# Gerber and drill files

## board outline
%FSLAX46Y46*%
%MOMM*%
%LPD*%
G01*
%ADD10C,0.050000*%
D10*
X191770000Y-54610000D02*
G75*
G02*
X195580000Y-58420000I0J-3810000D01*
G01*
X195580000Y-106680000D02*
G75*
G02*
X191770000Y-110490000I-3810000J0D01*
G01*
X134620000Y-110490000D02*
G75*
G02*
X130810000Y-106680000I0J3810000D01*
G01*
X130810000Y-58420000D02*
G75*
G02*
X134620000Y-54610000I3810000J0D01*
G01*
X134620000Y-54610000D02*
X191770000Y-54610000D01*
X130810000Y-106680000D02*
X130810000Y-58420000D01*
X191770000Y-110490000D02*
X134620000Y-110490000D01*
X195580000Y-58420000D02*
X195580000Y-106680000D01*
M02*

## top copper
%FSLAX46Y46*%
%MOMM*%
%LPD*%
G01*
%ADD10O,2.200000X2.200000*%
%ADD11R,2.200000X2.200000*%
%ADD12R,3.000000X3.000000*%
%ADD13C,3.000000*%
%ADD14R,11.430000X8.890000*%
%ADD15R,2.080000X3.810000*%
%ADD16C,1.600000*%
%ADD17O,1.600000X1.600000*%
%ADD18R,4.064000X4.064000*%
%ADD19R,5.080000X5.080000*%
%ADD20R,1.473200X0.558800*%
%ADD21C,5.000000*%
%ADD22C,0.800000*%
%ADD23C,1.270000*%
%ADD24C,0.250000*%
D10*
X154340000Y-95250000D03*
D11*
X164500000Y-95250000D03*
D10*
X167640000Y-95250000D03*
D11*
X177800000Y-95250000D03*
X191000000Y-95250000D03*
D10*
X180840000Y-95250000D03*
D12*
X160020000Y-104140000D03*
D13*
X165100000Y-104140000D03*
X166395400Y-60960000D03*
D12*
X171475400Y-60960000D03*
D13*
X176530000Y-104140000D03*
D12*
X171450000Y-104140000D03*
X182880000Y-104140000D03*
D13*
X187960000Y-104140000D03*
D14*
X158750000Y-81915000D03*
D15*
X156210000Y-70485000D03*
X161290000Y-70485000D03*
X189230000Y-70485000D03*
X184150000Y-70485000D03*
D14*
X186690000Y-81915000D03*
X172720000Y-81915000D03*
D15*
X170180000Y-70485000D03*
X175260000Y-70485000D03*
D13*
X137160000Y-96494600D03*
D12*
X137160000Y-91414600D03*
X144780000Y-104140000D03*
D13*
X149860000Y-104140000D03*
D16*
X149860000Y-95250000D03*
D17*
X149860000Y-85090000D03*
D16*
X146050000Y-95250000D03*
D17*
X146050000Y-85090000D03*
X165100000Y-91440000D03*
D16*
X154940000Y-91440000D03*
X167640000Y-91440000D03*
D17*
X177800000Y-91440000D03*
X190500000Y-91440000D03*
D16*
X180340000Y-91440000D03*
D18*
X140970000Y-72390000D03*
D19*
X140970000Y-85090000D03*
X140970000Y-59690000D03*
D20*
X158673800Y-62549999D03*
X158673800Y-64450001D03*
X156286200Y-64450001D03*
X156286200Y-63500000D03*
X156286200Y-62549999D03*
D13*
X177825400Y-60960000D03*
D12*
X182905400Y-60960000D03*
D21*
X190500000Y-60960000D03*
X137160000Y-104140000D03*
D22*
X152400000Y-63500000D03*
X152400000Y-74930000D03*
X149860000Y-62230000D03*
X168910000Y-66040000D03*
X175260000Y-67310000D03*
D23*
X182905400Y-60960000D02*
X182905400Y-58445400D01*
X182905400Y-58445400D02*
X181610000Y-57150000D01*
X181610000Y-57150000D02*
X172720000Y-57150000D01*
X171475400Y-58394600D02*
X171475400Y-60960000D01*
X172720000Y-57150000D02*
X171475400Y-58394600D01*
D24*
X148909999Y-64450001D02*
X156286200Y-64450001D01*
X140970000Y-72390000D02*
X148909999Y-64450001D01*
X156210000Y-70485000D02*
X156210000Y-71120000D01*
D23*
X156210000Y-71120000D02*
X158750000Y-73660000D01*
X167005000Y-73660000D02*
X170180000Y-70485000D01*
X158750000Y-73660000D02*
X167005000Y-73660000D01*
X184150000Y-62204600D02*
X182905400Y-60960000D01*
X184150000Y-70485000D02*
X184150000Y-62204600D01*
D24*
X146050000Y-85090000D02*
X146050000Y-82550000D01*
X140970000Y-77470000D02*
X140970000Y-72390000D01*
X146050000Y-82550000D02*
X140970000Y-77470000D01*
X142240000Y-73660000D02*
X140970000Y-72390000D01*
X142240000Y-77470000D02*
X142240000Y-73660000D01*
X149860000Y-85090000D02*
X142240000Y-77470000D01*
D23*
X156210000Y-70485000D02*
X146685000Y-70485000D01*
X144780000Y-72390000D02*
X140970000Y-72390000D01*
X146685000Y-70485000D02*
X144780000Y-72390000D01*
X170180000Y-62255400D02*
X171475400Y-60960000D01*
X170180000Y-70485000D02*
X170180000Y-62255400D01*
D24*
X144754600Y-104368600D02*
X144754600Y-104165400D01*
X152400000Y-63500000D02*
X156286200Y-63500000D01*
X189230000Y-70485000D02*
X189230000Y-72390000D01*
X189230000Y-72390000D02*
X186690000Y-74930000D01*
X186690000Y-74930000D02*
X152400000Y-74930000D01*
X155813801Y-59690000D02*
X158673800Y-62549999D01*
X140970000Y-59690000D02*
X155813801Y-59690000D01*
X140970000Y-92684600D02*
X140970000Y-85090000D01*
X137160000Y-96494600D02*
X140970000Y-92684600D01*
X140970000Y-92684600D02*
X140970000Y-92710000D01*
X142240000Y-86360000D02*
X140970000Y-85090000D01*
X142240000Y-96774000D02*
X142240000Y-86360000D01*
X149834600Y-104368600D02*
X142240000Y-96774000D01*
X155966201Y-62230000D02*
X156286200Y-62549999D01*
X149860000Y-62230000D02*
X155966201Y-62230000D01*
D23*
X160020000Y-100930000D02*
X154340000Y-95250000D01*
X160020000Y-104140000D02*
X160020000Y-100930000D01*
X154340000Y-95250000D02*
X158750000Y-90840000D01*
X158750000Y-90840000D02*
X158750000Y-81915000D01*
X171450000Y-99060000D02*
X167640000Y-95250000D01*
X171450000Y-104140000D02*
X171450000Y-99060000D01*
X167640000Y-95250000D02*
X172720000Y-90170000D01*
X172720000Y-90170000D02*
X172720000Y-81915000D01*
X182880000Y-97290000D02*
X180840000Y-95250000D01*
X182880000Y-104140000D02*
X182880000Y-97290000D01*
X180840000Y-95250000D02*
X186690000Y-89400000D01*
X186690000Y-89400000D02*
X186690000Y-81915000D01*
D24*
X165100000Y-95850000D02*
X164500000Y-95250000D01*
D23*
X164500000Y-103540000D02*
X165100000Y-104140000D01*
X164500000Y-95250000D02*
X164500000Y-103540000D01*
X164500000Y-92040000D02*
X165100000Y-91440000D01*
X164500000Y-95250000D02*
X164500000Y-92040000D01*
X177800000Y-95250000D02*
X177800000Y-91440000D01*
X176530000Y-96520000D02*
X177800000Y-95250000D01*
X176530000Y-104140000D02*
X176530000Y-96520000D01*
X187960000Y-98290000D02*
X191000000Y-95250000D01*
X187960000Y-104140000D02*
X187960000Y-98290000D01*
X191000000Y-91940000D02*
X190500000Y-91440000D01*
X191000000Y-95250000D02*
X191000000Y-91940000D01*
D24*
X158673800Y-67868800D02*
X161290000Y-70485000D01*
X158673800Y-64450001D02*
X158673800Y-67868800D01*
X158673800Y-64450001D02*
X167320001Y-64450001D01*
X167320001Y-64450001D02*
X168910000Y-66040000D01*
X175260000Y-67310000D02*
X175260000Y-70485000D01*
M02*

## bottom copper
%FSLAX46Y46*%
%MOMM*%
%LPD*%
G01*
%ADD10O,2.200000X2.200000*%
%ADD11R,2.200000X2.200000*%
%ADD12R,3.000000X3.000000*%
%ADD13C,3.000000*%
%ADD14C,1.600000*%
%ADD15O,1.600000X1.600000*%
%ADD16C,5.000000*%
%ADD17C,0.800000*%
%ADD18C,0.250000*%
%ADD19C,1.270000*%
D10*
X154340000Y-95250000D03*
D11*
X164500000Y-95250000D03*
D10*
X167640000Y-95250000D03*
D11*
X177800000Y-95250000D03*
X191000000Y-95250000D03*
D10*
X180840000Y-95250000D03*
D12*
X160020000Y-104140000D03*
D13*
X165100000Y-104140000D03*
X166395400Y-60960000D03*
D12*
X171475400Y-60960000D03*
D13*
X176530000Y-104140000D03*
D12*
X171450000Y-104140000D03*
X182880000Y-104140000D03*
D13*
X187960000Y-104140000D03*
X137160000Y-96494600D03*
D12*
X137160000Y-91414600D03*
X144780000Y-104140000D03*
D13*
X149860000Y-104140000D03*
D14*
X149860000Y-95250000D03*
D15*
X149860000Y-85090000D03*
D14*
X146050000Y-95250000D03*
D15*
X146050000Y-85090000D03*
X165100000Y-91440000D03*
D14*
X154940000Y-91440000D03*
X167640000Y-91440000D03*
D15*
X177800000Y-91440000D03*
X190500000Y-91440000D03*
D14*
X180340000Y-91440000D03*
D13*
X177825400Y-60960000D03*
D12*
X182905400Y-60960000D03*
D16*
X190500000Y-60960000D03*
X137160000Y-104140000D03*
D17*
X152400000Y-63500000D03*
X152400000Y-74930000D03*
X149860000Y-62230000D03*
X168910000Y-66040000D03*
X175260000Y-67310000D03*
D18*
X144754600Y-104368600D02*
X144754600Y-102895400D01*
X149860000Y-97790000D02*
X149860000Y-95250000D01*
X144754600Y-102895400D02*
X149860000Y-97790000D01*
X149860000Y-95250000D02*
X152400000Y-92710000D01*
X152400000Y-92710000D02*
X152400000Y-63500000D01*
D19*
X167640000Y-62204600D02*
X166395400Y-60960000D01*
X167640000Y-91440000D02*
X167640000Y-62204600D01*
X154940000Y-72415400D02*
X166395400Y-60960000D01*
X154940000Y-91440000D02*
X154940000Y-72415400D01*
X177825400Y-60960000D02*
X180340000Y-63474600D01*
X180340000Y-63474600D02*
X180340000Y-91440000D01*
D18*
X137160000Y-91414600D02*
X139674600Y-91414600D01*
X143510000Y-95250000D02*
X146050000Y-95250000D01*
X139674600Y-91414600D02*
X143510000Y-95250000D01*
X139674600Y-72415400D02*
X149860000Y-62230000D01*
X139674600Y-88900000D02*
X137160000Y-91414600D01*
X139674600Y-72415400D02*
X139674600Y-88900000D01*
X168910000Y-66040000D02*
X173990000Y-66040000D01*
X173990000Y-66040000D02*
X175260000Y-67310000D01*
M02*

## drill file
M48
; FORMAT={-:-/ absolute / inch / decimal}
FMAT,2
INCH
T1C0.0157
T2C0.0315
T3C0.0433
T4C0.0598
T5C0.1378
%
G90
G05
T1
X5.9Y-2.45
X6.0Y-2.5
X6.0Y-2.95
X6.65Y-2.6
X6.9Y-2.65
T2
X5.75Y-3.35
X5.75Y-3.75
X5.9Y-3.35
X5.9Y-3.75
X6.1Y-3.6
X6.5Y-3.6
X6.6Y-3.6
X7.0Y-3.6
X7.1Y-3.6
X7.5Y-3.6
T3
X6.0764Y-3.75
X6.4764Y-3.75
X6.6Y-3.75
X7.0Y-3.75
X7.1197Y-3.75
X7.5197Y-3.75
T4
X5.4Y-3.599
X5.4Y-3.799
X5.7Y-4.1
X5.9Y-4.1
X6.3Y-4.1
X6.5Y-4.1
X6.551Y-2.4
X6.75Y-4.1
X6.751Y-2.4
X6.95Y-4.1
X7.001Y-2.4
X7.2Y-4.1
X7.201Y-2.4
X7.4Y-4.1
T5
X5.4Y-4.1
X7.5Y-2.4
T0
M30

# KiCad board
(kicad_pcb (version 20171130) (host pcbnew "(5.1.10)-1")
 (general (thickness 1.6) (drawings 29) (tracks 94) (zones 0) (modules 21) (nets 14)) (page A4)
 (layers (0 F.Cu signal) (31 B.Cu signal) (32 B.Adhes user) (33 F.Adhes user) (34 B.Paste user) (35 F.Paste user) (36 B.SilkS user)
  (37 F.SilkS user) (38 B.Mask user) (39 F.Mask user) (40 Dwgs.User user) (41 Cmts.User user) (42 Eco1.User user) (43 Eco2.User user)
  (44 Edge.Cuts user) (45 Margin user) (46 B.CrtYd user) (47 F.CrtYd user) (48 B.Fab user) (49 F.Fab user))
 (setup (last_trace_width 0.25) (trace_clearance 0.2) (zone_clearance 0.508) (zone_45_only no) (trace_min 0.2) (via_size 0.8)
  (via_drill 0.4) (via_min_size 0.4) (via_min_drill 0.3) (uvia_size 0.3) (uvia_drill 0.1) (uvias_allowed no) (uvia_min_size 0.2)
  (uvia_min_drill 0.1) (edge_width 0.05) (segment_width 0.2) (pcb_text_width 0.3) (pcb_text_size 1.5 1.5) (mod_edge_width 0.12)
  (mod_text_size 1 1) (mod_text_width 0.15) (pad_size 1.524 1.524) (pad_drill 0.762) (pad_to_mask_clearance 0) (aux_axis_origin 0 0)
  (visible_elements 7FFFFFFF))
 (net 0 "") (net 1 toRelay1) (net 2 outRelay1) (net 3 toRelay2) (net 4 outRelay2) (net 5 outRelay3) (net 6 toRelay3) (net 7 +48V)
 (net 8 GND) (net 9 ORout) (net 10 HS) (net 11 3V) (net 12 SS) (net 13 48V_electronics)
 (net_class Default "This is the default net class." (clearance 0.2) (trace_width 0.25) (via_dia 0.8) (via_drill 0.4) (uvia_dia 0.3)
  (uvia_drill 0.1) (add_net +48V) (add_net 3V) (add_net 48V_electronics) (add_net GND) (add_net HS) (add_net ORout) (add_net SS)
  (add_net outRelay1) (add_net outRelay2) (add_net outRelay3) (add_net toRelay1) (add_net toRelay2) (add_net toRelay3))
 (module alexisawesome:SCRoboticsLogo (layer B.Cu) (at 172.72 78.74 180)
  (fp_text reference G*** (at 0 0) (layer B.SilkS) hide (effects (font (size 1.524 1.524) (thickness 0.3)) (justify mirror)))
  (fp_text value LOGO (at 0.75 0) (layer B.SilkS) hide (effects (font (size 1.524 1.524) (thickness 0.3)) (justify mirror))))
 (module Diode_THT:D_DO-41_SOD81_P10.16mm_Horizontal (layer F.Cu) (at 164.5 95.25 180)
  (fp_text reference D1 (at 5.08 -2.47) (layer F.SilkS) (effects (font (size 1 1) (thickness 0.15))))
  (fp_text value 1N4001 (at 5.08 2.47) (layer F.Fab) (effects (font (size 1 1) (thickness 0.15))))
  (pad 2 thru_hole oval (at 10.16 0 180) (size 2.2 2.2) (drill 1.1) (layers *.Cu *.Mask) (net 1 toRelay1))
  (pad 1 thru_hole rect (at 0 0 180) (size 2.2 2.2) (drill 1.1) (layers *.Cu *.Mask) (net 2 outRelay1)))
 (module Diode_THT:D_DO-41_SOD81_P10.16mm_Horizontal (layer F.Cu) (at 177.8 95.25 180)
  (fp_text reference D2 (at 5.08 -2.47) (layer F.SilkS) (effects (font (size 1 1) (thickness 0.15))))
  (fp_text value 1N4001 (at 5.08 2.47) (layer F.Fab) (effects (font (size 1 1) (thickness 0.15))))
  (pad 2 thru_hole oval (at 10.16 0 180) (size 2.2 2.2) (drill 1.1) (layers *.Cu *.Mask) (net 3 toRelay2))
  (pad 1 thru_hole rect (at 0 0 180) (size 2.2 2.2) (drill 1.1) (layers *.Cu *.Mask) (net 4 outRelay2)))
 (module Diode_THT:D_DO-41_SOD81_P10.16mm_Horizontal (layer F.Cu) (at 191 95.25 180)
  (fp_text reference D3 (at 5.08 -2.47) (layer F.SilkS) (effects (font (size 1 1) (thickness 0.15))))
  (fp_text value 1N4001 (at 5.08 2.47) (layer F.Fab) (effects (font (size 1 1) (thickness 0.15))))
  (pad 1 thru_hole rect (at 0 0 180) (size 2.2 2.2) (drill 1.1) (layers *.Cu *.Mask) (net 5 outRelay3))
  (pad 2 thru_hole oval (at 10.16 0 180) (size 2.2 2.2) (drill 1.1) (layers *.Cu *.Mask) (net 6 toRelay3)))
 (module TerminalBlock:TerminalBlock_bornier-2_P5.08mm (layer F.Cu) (at 160.02 104.14)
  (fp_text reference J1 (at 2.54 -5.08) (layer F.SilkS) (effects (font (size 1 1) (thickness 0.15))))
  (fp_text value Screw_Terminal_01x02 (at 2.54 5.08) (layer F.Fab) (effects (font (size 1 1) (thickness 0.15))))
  (pad 1 thru_hole rect (at 0 0) (size 3 3) (drill 1.52) (layers *.Cu *.Mask) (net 1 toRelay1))
  (pad 2 thru_hole circle (at 5.08 0) (size 3 3) (drill 1.52) (layers *.Cu *.Mask) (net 2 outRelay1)))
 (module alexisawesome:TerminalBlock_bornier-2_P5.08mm (layer F.Cu) (at 168.91 62.4586 180)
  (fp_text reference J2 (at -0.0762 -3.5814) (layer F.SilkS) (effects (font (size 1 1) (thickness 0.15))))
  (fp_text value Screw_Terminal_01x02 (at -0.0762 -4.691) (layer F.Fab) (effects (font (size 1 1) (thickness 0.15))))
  (pad 1 thru_hole circle (at 2.5146 1.4986 180) (size 3 3) (drill 1.52) (layers *.Cu *.Mask) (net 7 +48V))
  (pad 2 thru_hole rect (at -2.5654 1.4986 180) (size 3 3) (drill 1.52) (layers *.Cu *.Mask) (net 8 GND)))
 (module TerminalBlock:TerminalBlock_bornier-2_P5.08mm (layer F.Cu) (at 171.45 104.14)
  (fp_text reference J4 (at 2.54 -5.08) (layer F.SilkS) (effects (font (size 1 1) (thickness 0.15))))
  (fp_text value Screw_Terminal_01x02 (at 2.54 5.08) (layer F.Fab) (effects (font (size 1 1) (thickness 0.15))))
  (pad 2 thru_hole circle (at 5.08 0) (size 3 3) (drill 1.52) (layers *.Cu *.Mask) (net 4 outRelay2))
  (pad 1 thru_hole rect (at 0 0) (size 3 3) (drill 1.52) (layers *.Cu *.Mask) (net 3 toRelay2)))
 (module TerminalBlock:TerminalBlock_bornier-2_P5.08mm (layer F.Cu) (at 182.88 104.14)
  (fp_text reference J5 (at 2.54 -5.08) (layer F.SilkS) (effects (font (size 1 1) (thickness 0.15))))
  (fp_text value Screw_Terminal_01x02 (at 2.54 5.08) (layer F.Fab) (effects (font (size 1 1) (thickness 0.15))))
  (pad 1 thru_hole rect (at 0 0) (size 3 3) (drill 1.52) (layers *.Cu *.Mask) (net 6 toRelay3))
  (pad 2 thru_hole circle (at 5.08 0) (size 3 3) (drill 1.52) (layers *.Cu *.Mask) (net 5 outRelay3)))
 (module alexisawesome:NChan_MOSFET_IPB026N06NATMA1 (layer F.Cu) (at 158.75 77.47 180)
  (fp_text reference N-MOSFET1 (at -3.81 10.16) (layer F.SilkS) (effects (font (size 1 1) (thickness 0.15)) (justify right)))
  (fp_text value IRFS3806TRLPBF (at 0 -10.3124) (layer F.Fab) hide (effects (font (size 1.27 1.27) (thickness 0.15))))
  (pad 2 smd rect (at 0 -4.445 180) (size 11.43 8.89) (layers F.Cu F.Paste F.Mask) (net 1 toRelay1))
  (pad 3 smd rect (at 2.54 6.985 180) (size 2.08 3.81) (layers F.Cu F.Paste F.Mask) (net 8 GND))
  (pad 1 smd rect (at -2.54 6.985 180) (size 2.08 3.81) (layers F.Cu F.Paste F.Mask) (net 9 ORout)))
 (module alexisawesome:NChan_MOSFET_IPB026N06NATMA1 (layer F.Cu) (at 186.69 77.47 180)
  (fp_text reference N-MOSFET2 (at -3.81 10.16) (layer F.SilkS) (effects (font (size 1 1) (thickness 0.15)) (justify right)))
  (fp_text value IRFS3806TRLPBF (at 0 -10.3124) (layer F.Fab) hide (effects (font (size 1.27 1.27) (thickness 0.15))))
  (pad 1 smd rect (at -2.54 6.985 180) (size 2.08 3.81) (layers F.Cu F.Paste F.Mask) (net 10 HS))
  (pad 3 smd rect (at 2.54 6.985 180) (size 2.08 3.81) (layers F.Cu F.Paste F.Mask) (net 8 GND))
  (pad 2 smd rect (at 0 -4.445 180) (size 11.43 8.89) (layers F.Cu F.Paste F.Mask) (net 6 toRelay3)))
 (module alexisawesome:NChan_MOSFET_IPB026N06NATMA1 (layer F.Cu) (at 172.72 77.47 180)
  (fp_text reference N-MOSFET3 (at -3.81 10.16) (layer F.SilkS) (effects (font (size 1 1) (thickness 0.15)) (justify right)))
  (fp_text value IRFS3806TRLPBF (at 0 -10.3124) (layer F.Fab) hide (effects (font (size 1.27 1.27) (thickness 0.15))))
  (pad 2 smd rect (at 0 -4.445 180) (size 11.43 8.89) (layers F.Cu F.Paste F.Mask) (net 3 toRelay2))
  (pad 3 smd rect (at 2.54 6.985 180) (size 2.08 3.81) (layers F.Cu F.Paste F.Mask) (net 8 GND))
  (pad 1 smd rect (at -2.54 6.985 180) (size 2.08 3.81) (layers F.Cu F.Paste F.Mask) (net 9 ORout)))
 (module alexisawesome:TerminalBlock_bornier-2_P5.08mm (layer F.Cu) (at 138.6586 93.98 270)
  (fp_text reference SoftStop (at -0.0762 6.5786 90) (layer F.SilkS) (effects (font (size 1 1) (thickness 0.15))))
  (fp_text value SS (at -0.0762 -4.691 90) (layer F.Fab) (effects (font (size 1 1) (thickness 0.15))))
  (pad 1 thru_hole circle (at 2.5146 1.4986 270) (size 3 3) (drill 1.52) (layers *.Cu *.Mask) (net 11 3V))
  (pad 2 thru_hole rect (at -2.5654 1.4986 270) (size 3 3) (drill 1.52) (layers *.Cu *.Mask) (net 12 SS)))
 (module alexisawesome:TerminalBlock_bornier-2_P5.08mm (layer F.Cu) (at 147.3454 102.6414)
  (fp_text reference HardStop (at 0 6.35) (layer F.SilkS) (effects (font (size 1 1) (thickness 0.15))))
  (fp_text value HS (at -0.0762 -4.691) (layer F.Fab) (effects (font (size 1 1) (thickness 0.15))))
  (pad 2 thru_hole rect (at -2.5654 1.4986) (size 3 3) (drill 1.52) (layers *.Cu *.Mask) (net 10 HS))
  (pad 1 thru_hole circle (at 2.5146 1.4986) (size 3 3) (drill 1.52) (layers *.Cu *.Mask) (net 11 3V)))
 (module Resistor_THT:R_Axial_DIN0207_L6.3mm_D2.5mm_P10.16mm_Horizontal (layer F.Cu) (at 149.86 95.25 90)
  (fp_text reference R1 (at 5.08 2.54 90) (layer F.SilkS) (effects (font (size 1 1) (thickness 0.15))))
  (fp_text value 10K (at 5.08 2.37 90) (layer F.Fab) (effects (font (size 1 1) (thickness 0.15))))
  (pad 1 thru_hole circle (at 0 0 90) (size 1.6 1.6) (drill 0.8) (layers *.Cu *.Mask) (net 10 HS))
  (pad 2 thru_hole oval (at 10.16 0 90) (size 1.6 1.6) (drill 0.8) (layers *.Cu *.Mask) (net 8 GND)))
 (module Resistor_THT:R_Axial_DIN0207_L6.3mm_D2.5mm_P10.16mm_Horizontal (layer F.Cu) (at 146.05 95.25 90)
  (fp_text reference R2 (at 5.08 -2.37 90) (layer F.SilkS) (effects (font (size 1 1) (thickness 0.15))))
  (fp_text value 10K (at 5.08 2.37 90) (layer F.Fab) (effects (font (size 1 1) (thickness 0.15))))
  (pad 1 thru_hole circle (at 0 0 90) (size 1.6 1.6) (drill 0.8) (layers *.Cu *.Mask) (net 12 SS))
  (pad 2 thru_hole oval (at 10.16 0 90) (size 1.6 1.6) (drill 0.8) (layers *.Cu *.Mask) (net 8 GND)))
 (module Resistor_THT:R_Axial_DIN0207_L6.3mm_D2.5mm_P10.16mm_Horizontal (layer F.Cu) (at 154.94 91.44)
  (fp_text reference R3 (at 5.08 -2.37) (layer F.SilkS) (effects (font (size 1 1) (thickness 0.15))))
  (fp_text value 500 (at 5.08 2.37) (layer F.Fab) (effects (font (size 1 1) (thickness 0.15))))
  (pad 2 thru_hole oval (at 10.16 0) (size 1.6 1.6) (drill 0.8) (layers *.Cu *.Mask) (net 2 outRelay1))
  (pad 1 thru_hole circle (at 0 0) (size 1.6 1.6) (drill 0.8) (layers *.Cu *.Mask) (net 7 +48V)))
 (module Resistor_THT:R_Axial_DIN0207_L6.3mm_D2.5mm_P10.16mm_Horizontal (layer F.Cu) (at 167.64 91.44)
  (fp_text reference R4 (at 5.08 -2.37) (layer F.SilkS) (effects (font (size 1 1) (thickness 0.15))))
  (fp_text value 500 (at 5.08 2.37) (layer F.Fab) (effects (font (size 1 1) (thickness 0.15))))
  (pad 1 thru_hole circle (at 0 0) (size 1.6 1.6) (drill 0.8) (layers *.Cu *.Mask) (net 7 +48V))
  (pad 2 thru_hole oval (at 10.16 0) (size 1.6 1.6) (drill 0.8) (layers *.Cu *.Mask) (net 4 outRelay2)))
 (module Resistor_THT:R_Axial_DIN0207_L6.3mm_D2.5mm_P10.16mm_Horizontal (layer F.Cu) (at 180.34 91.44)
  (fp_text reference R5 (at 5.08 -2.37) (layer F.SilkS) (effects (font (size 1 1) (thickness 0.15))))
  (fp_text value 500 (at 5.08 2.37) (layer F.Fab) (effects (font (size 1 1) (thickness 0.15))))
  (pad 2 thru_hole oval (at 10.16 0) (size 1.6 1.6) (drill 0.8) (layers *.Cu *.Mask) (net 5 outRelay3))
  (pad 1 thru_hole circle (at 0 0) (size 1.6 1.6) (drill 0.8) (layers *.Cu *.Mask) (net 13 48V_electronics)))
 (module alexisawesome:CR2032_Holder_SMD (layer F.Cu) (at 140.97 72.39 90)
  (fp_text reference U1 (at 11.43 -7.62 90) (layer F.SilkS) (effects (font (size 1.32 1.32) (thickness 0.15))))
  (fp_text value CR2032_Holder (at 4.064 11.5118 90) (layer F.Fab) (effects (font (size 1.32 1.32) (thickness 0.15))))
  (pad - smd rect (at 0 0 90) (size 4.064 4.064) (layers F.Cu F.Paste F.Mask) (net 8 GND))
  (pad +$1 smd rect (at -12.7 0 90) (size 5.08 5.08) (layers F.Cu F.Paste F.Mask) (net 11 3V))
  (pad +$2 smd rect (at 12.7 0 90) (size 5.08 5.08) (layers F.Cu F.Paste F.Mask) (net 11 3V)))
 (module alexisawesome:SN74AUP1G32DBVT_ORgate (layer F.Cu) (at 157.48 63.5)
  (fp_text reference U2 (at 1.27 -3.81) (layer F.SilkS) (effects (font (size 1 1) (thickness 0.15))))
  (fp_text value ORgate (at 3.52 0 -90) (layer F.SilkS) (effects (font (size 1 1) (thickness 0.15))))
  (pad 5 smd rect (at 1.1938 -0.950001) (size 1.4732 0.5588) (layers F.Cu F.Paste F.Mask) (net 11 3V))
  (pad 4 smd rect (at 1.1938 0.950001) (size 1.4732 0.5588) (layers F.Cu F.Paste F.Mask) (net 9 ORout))
  (pad 3 smd rect (at -1.1938 0.950001) (size 1.4732 0.5588) (layers F.Cu F.Paste F.Mask) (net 8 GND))
  (pad 2 smd rect (at -1.1938 0) (size 1.4732 0.5588) (layers F.Cu F.Paste F.Mask) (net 10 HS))
  (pad 1 smd rect (at -1.1938 -0.950001) (size 1.4732 0.5588) (layers F.Cu F.Paste F.Mask) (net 12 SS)))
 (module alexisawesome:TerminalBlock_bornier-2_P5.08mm (layer F.Cu) (at 180.34 62.4586 180)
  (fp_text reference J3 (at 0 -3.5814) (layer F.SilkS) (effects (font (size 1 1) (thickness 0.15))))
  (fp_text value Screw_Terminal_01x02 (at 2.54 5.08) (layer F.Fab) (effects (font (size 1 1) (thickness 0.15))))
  (pad 1 thru_hole circle (at 2.5146 1.4986 180) (size 3 3) (drill 1.52) (layers *.Cu *.Mask) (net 13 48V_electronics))
  (pad 2 thru_hole rect (at -2.5654 1.4986 180) (size 3 3) (drill 1.52) (layers *.Cu *.Mask) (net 8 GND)))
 (gr_arc (start 191.77 58.42) (end 195.58 58.42) (angle -90) (layer Edge.Cuts) (width 0.05))
 (gr_arc (start 191.77 106.68) (end 191.77 110.49) (angle -90) (layer Edge.Cuts) (width 0.05))
 (gr_arc (start 134.62 106.68) (end 130.81 106.68) (angle -90) (layer Edge.Cuts) (width 0.05))
 (gr_arc (start 134.62 58.42) (end 134.62 54.61) (angle -90) (layer Edge.Cuts) (width 0.05))
 (gr_line (start 134.62 54.61) (end 191.77 54.61) (layer Edge.Cuts) (width 0.05))
 (gr_line (start 130.81 106.68) (end 130.81 58.42) (layer Edge.Cuts) (width 0.05))
 (gr_line (start 191.77 110.49) (end 134.62 110.49) (layer Edge.Cuts) (width 0.05))
 (gr_line (start 195.58 58.42) (end 195.58 106.68) (layer Edge.Cuts) (width 0.05))
 (via (at 190.5 60.96) (size 5) (drill 3.5) (layers F.Cu B.Cu) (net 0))
 (via (at 137.16 104.14) (size 5) (drill 3.5) (layers F.Cu B.Cu) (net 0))
 (segment (start 182.9054 60.96) (end 182.9054 58.4454) (width 1.27) (layer F.Cu) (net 8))
 (segment (start 182.9054 58.4454) (end 181.61 57.15) (width 1.27) (layer F.Cu) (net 8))
 (segment (start 181.61 57.15) (end 172.72 57.15) (width 1.27) (layer F.Cu) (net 8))
 (segment (start 171.4754 58.3946) (end 171.4754 60.96) (width 1.27) (layer F.Cu) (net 8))
 (segment (start 172.72 57.15) (end 171.4754 58.3946) (width 1.27) (layer F.Cu) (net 8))
 (segment (start 148.909999 64.450001) (end 156.2862 64.450001) (width 0.25) (layer F.Cu) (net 8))
 (segment (start 140.97 72.39) (end 148.909999 64.450001) (width 0.25) (layer F.Cu) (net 8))
 (segment (start 156.21 70.485) (end 156.21 71.12) (width 0.25) (layer F.Cu) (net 8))
 (segment (start 156.21 71.12) (end 158.75 73.66) (width 1.27) (layer F.Cu) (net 8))
 (segment (start 167.005 73.66) (end 170.18 70.485) (width 1.27) (layer F.Cu) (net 8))
 (segment (start 158.75 73.66) (end 167.005 73.66) (width 1.27) (layer F.Cu) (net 8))
 (segment (start 184.15 62.2046) (end 182.9054 60.96) (width 1.27) (layer F.Cu) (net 8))
 (segment (start 184.15 70.485) (end 184.15 62.2046) (width 1.27) (layer F.Cu) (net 8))
 (segment (start 146.05 85.09) (end 146.05 82.55) (width 0.25) (layer F.Cu) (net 8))
 (segment (start 140.97 77.47) (end 140.97 72.39) (width 0.25) (layer F.Cu) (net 8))
 (segment (start 146.05 82.55) (end 140.97 77.47) (width 0.25) (layer F.Cu) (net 8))
 (segment (start 142.24 73.66) (end 140.97 72.39) (width 0.25) (layer F.Cu) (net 8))
 (segment (start 142.24 77.47) (end 142.24 73.66) (width 0.25) (layer F.Cu) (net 8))
 (segment (start 149.86 85.09) (end 142.24 77.47) (width 0.25) (layer F.Cu) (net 8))
 (segment (start 156.21 70.485) (end 146.685 70.485) (width 1.27) (layer F.Cu) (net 8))
 (segment (start 144.78 72.39) (end 140.97 72.39) (width 1.27) (layer F.Cu) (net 8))
 (segment (start 146.685 70.485) (end 144.78 72.39) (width 1.27) (layer F.Cu) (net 8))
 (segment (start 170.18 62.2554) (end 171.4754 60.96) (width 1.27) (layer F.Cu) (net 8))
 (segment (start 170.18 70.485) (end 170.18 62.2554) (width 1.27) (layer F.Cu) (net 8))
 (segment (start 144.7546 104.3686) (end 144.7546 104.1654) (width 0.25) (layer F.Cu) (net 10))
 (segment (start 144.7546 104.3686) (end 144.7546 102.8954) (width 0.25) (layer B.Cu) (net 10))
 (segment (start 149.86 97.79) (end 149.86 95.25) (width 0.25) (layer B.Cu) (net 10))
 (segment (start 144.7546 102.8954) (end 149.86 97.79) (width 0.25) (layer B.Cu) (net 10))
 (segment (start 149.86 95.25) (end 152.4 92.71) (width 0.25) (layer B.Cu) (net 10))
 (segment (start 152.4 92.71) (end 152.4 63.5) (width 0.25) (layer B.Cu) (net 10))
 (via (at 152.4 63.5) (size 0.8) (drill 0.4) (layers F.Cu B.Cu) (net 10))
 (segment (start 152.4 63.5) (end 156.2862 63.5) (width 0.25) (layer F.Cu) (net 10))
 (segment (start 189.23 70.485) (end 189.23 72.39) (width 0.25) (layer F.Cu) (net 10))
 (segment (start 189.23 72.39) (end 186.69 74.93) (width 0.25) (layer F.Cu) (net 10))
 (segment (start 186.69 74.93) (end 152.4 74.93) (width 0.25) (layer F.Cu) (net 10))
 (via (at 152.4 74.93) (size 0.8) (drill 0.4) (layers F.Cu B.Cu) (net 10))
 (segment (start 167.64 62.2046) (end 166.3954 60.96) (width 1.27) (layer B.Cu) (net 7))
 (segment (start 167.64 91.44) (end 167.64 62.2046) (width 1.27) (layer B.Cu) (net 7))
 (segment (start 154.94 72.4154) (end 166.3954 60.96) (width 1.27) (layer B.Cu) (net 7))
 (segment (start 154.94 91.44) (end 154.94 72.4154) (width 1.27) (layer B.Cu) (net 7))
 (segment (start 177.8254 60.96) (end 180.34 63.4746) (width 1.27) (layer B.Cu) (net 13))
 (segment (start 180.34 63.4746) (end 180.34 91.44) (width 1.27) (layer B.Cu) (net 13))
 (segment (start 155.813801 59.69) (end 158.6738 62.549999) (width 0.25) (layer F.Cu) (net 11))
 (segment (start 140.97 59.69) (end 155.813801 59.69) (width 0.25) (layer F.Cu) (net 11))
 (segment (start 140.97 92.6846) (end 140.97 85.09) (width 0.25) (layer F.Cu) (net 11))
 (segment (start 137.16 96.4946) (end 140.97 92.6846) (width 0.25) (layer F.Cu) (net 11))
 (segment (start 140.97 92.6846) (end 140.97 92.71) (width 0.25) (layer F.Cu) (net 11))
 (segment (start 142.24 86.36) (end 140.97 85.09) (width 0.25) (layer F.Cu) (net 11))
 (segment (start 142.24 96.774) (end 142.24 86.36) (width 0.25) (layer F.Cu) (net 11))
 (segment (start 149.8346 104.3686) (end 142.24 96.774) (width 0.25) (layer F.Cu) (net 11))
 (segment (start 137.16 91.4146) (end 139.6746 91.4146) (width 0.25) (layer B.Cu) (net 12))
 (segment (start 143.51 95.25) (end 146.05 95.25) (width 0.25) (layer B.Cu) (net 12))
 (segment (start 139.6746 91.4146) (end 143.51 95.25) (width 0.25) (layer B.Cu) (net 12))
 (segment (start 139.6746 72.4154) (end 149.86 62.23) (width 0.25) (layer B.Cu) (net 12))
 (via (at 149.86 62.23) (size 0.8) (drill 0.4) (layers F.Cu B.Cu) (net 12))
 (segment (start 155.966201 62.23) (end 156.2862 62.549999) (width 0.25) (layer F.Cu) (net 12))
 (segment (start 149.86 62.23) (end 155.966201 62.23) (width 0.25) (layer F.Cu) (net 12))
 (segment (start 139.6746 88.9) (end 137.16 91.4146) (width 0.25) (layer B.Cu) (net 12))
 (segment (start 139.6746 72.4154) (end 139.6746 88.9) (width 0.25) (layer B.Cu) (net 12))
 (segment (start 160.02 100.93) (end 154.34 95.25) (width 1.27) (layer F.Cu) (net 1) (status 20))
 (segment (start 160.02 104.14) (end 160.02 100.93) (width 1.27) (layer F.Cu) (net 1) (status 10))
 (segment (start 154.34 95.25) (end 158.75 90.84) (width 1.27) (layer F.Cu) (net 1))
 (segment (start 158.75 90.84) (end 158.75 81.915) (width 1.27) (layer F.Cu) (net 1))
 (segment (start 171.45 99.06) (end 167.64 95.25) (width 1.27) (layer F.Cu) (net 3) (status 20))
 (segment (start 171.45 104.14) (end 171.45 99.06) (width 1.27) (layer F.Cu) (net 3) (status 10))
 (segment (start 167.64 95.25) (end 172.72 90.17) (width 1.27) (layer F.Cu) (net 3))
 (segment (start 172.72 90.17) (end 172.72 81.915) (width 1.27) (layer F.Cu) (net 3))
 (segment (start 182.88 97.29) (end 180.84 95.25) (width 1.27) (layer F.Cu) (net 6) (status 20))
 (segment (start 182.88 104.14) (end 182.88 97.29) (width 1.27) (layer F.Cu) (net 6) (status 10))
 (segment (start 180.84 95.25) (end 186.69 89.4) (width 1.27) (layer F.Cu) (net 6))
 (segment (start 186.69 89.4) (end 186.69 81.915) (width 1.27) (layer F.Cu) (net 6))
 (segment (start 165.1 95.85) (end 164.5 95.25) (width 0.25) (layer F.Cu) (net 2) (status 30))
 (segment (start 164.5 103.54) (end 165.1 104.14) (width 1.27) (layer F.Cu) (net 2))
 (segment (start 164.5 95.25) (end 164.5 103.54) (width 1.27) (layer F.Cu) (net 2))
 (segment (start 164.5 92.04) (end 165.1 91.44) (width 1.27) (layer F.Cu) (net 2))
 (segment (start 164.5 95.25) (end 164.5 92.04) (width 1.27) (layer F.Cu) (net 2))
 (segment (start 177.8 95.25) (end 177.8 91.44) (width 1.27) (layer F.Cu) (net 4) (status 30))
 (segment (start 176.53 96.52) (end 177.8 95.25) (width 1.27) (layer F.Cu) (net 4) (status 20))
 (segment (start 176.53 104.14) (end 176.53 96.52) (width 1.27) (layer F.Cu) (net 4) (status 10))
 (segment (start 187.96 98.29) (end 191 95.25) (width 1.27) (layer F.Cu) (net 5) (status 20))
 (segment (start 187.96 104.14) (end 187.96 98.29) (width 1.27) (layer F.Cu) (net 5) (status 10))
 (segment (start 191 91.94) (end 190.5 91.44) (width 1.27) (layer F.Cu) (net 5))
 (segment (start 191 95.25) (end 191 91.94) (width 1.27) (layer F.Cu) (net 5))
 (segment (start 158.6738 67.8688) (end 161.29 70.485) (width 0.25) (layer F.Cu) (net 9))
 (segment (start 158.6738 64.450001) (end 158.6738 67.8688) (width 0.25) (layer F.Cu) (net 9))
 (segment (start 158.6738 64.450001) (end 167.320001 64.450001) (width 0.25) (layer F.Cu) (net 9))
 (segment (start 167.320001 64.450001) (end 168.91 66.04) (width 0.25) (layer F.Cu) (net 9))
 (via (at 168.91 66.04) (size 0.8) (drill 0.4) (layers F.Cu B.Cu) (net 9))
 (segment (start 168.91 66.04) (end 173.99 66.04) (width 0.25) (layer B.Cu) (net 9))
 (segment (start 173.99 66.04) (end 175.26 67.31) (width 0.25) (layer B.Cu) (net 9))
 (via (at 175.26 67.31) (size 0.8) (drill 0.4) (layers F.Cu B.Cu) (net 9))
 (segment (start 175.26 67.31) (end 175.26 70.485) (width 0.25) (layer F.Cu) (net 9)))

